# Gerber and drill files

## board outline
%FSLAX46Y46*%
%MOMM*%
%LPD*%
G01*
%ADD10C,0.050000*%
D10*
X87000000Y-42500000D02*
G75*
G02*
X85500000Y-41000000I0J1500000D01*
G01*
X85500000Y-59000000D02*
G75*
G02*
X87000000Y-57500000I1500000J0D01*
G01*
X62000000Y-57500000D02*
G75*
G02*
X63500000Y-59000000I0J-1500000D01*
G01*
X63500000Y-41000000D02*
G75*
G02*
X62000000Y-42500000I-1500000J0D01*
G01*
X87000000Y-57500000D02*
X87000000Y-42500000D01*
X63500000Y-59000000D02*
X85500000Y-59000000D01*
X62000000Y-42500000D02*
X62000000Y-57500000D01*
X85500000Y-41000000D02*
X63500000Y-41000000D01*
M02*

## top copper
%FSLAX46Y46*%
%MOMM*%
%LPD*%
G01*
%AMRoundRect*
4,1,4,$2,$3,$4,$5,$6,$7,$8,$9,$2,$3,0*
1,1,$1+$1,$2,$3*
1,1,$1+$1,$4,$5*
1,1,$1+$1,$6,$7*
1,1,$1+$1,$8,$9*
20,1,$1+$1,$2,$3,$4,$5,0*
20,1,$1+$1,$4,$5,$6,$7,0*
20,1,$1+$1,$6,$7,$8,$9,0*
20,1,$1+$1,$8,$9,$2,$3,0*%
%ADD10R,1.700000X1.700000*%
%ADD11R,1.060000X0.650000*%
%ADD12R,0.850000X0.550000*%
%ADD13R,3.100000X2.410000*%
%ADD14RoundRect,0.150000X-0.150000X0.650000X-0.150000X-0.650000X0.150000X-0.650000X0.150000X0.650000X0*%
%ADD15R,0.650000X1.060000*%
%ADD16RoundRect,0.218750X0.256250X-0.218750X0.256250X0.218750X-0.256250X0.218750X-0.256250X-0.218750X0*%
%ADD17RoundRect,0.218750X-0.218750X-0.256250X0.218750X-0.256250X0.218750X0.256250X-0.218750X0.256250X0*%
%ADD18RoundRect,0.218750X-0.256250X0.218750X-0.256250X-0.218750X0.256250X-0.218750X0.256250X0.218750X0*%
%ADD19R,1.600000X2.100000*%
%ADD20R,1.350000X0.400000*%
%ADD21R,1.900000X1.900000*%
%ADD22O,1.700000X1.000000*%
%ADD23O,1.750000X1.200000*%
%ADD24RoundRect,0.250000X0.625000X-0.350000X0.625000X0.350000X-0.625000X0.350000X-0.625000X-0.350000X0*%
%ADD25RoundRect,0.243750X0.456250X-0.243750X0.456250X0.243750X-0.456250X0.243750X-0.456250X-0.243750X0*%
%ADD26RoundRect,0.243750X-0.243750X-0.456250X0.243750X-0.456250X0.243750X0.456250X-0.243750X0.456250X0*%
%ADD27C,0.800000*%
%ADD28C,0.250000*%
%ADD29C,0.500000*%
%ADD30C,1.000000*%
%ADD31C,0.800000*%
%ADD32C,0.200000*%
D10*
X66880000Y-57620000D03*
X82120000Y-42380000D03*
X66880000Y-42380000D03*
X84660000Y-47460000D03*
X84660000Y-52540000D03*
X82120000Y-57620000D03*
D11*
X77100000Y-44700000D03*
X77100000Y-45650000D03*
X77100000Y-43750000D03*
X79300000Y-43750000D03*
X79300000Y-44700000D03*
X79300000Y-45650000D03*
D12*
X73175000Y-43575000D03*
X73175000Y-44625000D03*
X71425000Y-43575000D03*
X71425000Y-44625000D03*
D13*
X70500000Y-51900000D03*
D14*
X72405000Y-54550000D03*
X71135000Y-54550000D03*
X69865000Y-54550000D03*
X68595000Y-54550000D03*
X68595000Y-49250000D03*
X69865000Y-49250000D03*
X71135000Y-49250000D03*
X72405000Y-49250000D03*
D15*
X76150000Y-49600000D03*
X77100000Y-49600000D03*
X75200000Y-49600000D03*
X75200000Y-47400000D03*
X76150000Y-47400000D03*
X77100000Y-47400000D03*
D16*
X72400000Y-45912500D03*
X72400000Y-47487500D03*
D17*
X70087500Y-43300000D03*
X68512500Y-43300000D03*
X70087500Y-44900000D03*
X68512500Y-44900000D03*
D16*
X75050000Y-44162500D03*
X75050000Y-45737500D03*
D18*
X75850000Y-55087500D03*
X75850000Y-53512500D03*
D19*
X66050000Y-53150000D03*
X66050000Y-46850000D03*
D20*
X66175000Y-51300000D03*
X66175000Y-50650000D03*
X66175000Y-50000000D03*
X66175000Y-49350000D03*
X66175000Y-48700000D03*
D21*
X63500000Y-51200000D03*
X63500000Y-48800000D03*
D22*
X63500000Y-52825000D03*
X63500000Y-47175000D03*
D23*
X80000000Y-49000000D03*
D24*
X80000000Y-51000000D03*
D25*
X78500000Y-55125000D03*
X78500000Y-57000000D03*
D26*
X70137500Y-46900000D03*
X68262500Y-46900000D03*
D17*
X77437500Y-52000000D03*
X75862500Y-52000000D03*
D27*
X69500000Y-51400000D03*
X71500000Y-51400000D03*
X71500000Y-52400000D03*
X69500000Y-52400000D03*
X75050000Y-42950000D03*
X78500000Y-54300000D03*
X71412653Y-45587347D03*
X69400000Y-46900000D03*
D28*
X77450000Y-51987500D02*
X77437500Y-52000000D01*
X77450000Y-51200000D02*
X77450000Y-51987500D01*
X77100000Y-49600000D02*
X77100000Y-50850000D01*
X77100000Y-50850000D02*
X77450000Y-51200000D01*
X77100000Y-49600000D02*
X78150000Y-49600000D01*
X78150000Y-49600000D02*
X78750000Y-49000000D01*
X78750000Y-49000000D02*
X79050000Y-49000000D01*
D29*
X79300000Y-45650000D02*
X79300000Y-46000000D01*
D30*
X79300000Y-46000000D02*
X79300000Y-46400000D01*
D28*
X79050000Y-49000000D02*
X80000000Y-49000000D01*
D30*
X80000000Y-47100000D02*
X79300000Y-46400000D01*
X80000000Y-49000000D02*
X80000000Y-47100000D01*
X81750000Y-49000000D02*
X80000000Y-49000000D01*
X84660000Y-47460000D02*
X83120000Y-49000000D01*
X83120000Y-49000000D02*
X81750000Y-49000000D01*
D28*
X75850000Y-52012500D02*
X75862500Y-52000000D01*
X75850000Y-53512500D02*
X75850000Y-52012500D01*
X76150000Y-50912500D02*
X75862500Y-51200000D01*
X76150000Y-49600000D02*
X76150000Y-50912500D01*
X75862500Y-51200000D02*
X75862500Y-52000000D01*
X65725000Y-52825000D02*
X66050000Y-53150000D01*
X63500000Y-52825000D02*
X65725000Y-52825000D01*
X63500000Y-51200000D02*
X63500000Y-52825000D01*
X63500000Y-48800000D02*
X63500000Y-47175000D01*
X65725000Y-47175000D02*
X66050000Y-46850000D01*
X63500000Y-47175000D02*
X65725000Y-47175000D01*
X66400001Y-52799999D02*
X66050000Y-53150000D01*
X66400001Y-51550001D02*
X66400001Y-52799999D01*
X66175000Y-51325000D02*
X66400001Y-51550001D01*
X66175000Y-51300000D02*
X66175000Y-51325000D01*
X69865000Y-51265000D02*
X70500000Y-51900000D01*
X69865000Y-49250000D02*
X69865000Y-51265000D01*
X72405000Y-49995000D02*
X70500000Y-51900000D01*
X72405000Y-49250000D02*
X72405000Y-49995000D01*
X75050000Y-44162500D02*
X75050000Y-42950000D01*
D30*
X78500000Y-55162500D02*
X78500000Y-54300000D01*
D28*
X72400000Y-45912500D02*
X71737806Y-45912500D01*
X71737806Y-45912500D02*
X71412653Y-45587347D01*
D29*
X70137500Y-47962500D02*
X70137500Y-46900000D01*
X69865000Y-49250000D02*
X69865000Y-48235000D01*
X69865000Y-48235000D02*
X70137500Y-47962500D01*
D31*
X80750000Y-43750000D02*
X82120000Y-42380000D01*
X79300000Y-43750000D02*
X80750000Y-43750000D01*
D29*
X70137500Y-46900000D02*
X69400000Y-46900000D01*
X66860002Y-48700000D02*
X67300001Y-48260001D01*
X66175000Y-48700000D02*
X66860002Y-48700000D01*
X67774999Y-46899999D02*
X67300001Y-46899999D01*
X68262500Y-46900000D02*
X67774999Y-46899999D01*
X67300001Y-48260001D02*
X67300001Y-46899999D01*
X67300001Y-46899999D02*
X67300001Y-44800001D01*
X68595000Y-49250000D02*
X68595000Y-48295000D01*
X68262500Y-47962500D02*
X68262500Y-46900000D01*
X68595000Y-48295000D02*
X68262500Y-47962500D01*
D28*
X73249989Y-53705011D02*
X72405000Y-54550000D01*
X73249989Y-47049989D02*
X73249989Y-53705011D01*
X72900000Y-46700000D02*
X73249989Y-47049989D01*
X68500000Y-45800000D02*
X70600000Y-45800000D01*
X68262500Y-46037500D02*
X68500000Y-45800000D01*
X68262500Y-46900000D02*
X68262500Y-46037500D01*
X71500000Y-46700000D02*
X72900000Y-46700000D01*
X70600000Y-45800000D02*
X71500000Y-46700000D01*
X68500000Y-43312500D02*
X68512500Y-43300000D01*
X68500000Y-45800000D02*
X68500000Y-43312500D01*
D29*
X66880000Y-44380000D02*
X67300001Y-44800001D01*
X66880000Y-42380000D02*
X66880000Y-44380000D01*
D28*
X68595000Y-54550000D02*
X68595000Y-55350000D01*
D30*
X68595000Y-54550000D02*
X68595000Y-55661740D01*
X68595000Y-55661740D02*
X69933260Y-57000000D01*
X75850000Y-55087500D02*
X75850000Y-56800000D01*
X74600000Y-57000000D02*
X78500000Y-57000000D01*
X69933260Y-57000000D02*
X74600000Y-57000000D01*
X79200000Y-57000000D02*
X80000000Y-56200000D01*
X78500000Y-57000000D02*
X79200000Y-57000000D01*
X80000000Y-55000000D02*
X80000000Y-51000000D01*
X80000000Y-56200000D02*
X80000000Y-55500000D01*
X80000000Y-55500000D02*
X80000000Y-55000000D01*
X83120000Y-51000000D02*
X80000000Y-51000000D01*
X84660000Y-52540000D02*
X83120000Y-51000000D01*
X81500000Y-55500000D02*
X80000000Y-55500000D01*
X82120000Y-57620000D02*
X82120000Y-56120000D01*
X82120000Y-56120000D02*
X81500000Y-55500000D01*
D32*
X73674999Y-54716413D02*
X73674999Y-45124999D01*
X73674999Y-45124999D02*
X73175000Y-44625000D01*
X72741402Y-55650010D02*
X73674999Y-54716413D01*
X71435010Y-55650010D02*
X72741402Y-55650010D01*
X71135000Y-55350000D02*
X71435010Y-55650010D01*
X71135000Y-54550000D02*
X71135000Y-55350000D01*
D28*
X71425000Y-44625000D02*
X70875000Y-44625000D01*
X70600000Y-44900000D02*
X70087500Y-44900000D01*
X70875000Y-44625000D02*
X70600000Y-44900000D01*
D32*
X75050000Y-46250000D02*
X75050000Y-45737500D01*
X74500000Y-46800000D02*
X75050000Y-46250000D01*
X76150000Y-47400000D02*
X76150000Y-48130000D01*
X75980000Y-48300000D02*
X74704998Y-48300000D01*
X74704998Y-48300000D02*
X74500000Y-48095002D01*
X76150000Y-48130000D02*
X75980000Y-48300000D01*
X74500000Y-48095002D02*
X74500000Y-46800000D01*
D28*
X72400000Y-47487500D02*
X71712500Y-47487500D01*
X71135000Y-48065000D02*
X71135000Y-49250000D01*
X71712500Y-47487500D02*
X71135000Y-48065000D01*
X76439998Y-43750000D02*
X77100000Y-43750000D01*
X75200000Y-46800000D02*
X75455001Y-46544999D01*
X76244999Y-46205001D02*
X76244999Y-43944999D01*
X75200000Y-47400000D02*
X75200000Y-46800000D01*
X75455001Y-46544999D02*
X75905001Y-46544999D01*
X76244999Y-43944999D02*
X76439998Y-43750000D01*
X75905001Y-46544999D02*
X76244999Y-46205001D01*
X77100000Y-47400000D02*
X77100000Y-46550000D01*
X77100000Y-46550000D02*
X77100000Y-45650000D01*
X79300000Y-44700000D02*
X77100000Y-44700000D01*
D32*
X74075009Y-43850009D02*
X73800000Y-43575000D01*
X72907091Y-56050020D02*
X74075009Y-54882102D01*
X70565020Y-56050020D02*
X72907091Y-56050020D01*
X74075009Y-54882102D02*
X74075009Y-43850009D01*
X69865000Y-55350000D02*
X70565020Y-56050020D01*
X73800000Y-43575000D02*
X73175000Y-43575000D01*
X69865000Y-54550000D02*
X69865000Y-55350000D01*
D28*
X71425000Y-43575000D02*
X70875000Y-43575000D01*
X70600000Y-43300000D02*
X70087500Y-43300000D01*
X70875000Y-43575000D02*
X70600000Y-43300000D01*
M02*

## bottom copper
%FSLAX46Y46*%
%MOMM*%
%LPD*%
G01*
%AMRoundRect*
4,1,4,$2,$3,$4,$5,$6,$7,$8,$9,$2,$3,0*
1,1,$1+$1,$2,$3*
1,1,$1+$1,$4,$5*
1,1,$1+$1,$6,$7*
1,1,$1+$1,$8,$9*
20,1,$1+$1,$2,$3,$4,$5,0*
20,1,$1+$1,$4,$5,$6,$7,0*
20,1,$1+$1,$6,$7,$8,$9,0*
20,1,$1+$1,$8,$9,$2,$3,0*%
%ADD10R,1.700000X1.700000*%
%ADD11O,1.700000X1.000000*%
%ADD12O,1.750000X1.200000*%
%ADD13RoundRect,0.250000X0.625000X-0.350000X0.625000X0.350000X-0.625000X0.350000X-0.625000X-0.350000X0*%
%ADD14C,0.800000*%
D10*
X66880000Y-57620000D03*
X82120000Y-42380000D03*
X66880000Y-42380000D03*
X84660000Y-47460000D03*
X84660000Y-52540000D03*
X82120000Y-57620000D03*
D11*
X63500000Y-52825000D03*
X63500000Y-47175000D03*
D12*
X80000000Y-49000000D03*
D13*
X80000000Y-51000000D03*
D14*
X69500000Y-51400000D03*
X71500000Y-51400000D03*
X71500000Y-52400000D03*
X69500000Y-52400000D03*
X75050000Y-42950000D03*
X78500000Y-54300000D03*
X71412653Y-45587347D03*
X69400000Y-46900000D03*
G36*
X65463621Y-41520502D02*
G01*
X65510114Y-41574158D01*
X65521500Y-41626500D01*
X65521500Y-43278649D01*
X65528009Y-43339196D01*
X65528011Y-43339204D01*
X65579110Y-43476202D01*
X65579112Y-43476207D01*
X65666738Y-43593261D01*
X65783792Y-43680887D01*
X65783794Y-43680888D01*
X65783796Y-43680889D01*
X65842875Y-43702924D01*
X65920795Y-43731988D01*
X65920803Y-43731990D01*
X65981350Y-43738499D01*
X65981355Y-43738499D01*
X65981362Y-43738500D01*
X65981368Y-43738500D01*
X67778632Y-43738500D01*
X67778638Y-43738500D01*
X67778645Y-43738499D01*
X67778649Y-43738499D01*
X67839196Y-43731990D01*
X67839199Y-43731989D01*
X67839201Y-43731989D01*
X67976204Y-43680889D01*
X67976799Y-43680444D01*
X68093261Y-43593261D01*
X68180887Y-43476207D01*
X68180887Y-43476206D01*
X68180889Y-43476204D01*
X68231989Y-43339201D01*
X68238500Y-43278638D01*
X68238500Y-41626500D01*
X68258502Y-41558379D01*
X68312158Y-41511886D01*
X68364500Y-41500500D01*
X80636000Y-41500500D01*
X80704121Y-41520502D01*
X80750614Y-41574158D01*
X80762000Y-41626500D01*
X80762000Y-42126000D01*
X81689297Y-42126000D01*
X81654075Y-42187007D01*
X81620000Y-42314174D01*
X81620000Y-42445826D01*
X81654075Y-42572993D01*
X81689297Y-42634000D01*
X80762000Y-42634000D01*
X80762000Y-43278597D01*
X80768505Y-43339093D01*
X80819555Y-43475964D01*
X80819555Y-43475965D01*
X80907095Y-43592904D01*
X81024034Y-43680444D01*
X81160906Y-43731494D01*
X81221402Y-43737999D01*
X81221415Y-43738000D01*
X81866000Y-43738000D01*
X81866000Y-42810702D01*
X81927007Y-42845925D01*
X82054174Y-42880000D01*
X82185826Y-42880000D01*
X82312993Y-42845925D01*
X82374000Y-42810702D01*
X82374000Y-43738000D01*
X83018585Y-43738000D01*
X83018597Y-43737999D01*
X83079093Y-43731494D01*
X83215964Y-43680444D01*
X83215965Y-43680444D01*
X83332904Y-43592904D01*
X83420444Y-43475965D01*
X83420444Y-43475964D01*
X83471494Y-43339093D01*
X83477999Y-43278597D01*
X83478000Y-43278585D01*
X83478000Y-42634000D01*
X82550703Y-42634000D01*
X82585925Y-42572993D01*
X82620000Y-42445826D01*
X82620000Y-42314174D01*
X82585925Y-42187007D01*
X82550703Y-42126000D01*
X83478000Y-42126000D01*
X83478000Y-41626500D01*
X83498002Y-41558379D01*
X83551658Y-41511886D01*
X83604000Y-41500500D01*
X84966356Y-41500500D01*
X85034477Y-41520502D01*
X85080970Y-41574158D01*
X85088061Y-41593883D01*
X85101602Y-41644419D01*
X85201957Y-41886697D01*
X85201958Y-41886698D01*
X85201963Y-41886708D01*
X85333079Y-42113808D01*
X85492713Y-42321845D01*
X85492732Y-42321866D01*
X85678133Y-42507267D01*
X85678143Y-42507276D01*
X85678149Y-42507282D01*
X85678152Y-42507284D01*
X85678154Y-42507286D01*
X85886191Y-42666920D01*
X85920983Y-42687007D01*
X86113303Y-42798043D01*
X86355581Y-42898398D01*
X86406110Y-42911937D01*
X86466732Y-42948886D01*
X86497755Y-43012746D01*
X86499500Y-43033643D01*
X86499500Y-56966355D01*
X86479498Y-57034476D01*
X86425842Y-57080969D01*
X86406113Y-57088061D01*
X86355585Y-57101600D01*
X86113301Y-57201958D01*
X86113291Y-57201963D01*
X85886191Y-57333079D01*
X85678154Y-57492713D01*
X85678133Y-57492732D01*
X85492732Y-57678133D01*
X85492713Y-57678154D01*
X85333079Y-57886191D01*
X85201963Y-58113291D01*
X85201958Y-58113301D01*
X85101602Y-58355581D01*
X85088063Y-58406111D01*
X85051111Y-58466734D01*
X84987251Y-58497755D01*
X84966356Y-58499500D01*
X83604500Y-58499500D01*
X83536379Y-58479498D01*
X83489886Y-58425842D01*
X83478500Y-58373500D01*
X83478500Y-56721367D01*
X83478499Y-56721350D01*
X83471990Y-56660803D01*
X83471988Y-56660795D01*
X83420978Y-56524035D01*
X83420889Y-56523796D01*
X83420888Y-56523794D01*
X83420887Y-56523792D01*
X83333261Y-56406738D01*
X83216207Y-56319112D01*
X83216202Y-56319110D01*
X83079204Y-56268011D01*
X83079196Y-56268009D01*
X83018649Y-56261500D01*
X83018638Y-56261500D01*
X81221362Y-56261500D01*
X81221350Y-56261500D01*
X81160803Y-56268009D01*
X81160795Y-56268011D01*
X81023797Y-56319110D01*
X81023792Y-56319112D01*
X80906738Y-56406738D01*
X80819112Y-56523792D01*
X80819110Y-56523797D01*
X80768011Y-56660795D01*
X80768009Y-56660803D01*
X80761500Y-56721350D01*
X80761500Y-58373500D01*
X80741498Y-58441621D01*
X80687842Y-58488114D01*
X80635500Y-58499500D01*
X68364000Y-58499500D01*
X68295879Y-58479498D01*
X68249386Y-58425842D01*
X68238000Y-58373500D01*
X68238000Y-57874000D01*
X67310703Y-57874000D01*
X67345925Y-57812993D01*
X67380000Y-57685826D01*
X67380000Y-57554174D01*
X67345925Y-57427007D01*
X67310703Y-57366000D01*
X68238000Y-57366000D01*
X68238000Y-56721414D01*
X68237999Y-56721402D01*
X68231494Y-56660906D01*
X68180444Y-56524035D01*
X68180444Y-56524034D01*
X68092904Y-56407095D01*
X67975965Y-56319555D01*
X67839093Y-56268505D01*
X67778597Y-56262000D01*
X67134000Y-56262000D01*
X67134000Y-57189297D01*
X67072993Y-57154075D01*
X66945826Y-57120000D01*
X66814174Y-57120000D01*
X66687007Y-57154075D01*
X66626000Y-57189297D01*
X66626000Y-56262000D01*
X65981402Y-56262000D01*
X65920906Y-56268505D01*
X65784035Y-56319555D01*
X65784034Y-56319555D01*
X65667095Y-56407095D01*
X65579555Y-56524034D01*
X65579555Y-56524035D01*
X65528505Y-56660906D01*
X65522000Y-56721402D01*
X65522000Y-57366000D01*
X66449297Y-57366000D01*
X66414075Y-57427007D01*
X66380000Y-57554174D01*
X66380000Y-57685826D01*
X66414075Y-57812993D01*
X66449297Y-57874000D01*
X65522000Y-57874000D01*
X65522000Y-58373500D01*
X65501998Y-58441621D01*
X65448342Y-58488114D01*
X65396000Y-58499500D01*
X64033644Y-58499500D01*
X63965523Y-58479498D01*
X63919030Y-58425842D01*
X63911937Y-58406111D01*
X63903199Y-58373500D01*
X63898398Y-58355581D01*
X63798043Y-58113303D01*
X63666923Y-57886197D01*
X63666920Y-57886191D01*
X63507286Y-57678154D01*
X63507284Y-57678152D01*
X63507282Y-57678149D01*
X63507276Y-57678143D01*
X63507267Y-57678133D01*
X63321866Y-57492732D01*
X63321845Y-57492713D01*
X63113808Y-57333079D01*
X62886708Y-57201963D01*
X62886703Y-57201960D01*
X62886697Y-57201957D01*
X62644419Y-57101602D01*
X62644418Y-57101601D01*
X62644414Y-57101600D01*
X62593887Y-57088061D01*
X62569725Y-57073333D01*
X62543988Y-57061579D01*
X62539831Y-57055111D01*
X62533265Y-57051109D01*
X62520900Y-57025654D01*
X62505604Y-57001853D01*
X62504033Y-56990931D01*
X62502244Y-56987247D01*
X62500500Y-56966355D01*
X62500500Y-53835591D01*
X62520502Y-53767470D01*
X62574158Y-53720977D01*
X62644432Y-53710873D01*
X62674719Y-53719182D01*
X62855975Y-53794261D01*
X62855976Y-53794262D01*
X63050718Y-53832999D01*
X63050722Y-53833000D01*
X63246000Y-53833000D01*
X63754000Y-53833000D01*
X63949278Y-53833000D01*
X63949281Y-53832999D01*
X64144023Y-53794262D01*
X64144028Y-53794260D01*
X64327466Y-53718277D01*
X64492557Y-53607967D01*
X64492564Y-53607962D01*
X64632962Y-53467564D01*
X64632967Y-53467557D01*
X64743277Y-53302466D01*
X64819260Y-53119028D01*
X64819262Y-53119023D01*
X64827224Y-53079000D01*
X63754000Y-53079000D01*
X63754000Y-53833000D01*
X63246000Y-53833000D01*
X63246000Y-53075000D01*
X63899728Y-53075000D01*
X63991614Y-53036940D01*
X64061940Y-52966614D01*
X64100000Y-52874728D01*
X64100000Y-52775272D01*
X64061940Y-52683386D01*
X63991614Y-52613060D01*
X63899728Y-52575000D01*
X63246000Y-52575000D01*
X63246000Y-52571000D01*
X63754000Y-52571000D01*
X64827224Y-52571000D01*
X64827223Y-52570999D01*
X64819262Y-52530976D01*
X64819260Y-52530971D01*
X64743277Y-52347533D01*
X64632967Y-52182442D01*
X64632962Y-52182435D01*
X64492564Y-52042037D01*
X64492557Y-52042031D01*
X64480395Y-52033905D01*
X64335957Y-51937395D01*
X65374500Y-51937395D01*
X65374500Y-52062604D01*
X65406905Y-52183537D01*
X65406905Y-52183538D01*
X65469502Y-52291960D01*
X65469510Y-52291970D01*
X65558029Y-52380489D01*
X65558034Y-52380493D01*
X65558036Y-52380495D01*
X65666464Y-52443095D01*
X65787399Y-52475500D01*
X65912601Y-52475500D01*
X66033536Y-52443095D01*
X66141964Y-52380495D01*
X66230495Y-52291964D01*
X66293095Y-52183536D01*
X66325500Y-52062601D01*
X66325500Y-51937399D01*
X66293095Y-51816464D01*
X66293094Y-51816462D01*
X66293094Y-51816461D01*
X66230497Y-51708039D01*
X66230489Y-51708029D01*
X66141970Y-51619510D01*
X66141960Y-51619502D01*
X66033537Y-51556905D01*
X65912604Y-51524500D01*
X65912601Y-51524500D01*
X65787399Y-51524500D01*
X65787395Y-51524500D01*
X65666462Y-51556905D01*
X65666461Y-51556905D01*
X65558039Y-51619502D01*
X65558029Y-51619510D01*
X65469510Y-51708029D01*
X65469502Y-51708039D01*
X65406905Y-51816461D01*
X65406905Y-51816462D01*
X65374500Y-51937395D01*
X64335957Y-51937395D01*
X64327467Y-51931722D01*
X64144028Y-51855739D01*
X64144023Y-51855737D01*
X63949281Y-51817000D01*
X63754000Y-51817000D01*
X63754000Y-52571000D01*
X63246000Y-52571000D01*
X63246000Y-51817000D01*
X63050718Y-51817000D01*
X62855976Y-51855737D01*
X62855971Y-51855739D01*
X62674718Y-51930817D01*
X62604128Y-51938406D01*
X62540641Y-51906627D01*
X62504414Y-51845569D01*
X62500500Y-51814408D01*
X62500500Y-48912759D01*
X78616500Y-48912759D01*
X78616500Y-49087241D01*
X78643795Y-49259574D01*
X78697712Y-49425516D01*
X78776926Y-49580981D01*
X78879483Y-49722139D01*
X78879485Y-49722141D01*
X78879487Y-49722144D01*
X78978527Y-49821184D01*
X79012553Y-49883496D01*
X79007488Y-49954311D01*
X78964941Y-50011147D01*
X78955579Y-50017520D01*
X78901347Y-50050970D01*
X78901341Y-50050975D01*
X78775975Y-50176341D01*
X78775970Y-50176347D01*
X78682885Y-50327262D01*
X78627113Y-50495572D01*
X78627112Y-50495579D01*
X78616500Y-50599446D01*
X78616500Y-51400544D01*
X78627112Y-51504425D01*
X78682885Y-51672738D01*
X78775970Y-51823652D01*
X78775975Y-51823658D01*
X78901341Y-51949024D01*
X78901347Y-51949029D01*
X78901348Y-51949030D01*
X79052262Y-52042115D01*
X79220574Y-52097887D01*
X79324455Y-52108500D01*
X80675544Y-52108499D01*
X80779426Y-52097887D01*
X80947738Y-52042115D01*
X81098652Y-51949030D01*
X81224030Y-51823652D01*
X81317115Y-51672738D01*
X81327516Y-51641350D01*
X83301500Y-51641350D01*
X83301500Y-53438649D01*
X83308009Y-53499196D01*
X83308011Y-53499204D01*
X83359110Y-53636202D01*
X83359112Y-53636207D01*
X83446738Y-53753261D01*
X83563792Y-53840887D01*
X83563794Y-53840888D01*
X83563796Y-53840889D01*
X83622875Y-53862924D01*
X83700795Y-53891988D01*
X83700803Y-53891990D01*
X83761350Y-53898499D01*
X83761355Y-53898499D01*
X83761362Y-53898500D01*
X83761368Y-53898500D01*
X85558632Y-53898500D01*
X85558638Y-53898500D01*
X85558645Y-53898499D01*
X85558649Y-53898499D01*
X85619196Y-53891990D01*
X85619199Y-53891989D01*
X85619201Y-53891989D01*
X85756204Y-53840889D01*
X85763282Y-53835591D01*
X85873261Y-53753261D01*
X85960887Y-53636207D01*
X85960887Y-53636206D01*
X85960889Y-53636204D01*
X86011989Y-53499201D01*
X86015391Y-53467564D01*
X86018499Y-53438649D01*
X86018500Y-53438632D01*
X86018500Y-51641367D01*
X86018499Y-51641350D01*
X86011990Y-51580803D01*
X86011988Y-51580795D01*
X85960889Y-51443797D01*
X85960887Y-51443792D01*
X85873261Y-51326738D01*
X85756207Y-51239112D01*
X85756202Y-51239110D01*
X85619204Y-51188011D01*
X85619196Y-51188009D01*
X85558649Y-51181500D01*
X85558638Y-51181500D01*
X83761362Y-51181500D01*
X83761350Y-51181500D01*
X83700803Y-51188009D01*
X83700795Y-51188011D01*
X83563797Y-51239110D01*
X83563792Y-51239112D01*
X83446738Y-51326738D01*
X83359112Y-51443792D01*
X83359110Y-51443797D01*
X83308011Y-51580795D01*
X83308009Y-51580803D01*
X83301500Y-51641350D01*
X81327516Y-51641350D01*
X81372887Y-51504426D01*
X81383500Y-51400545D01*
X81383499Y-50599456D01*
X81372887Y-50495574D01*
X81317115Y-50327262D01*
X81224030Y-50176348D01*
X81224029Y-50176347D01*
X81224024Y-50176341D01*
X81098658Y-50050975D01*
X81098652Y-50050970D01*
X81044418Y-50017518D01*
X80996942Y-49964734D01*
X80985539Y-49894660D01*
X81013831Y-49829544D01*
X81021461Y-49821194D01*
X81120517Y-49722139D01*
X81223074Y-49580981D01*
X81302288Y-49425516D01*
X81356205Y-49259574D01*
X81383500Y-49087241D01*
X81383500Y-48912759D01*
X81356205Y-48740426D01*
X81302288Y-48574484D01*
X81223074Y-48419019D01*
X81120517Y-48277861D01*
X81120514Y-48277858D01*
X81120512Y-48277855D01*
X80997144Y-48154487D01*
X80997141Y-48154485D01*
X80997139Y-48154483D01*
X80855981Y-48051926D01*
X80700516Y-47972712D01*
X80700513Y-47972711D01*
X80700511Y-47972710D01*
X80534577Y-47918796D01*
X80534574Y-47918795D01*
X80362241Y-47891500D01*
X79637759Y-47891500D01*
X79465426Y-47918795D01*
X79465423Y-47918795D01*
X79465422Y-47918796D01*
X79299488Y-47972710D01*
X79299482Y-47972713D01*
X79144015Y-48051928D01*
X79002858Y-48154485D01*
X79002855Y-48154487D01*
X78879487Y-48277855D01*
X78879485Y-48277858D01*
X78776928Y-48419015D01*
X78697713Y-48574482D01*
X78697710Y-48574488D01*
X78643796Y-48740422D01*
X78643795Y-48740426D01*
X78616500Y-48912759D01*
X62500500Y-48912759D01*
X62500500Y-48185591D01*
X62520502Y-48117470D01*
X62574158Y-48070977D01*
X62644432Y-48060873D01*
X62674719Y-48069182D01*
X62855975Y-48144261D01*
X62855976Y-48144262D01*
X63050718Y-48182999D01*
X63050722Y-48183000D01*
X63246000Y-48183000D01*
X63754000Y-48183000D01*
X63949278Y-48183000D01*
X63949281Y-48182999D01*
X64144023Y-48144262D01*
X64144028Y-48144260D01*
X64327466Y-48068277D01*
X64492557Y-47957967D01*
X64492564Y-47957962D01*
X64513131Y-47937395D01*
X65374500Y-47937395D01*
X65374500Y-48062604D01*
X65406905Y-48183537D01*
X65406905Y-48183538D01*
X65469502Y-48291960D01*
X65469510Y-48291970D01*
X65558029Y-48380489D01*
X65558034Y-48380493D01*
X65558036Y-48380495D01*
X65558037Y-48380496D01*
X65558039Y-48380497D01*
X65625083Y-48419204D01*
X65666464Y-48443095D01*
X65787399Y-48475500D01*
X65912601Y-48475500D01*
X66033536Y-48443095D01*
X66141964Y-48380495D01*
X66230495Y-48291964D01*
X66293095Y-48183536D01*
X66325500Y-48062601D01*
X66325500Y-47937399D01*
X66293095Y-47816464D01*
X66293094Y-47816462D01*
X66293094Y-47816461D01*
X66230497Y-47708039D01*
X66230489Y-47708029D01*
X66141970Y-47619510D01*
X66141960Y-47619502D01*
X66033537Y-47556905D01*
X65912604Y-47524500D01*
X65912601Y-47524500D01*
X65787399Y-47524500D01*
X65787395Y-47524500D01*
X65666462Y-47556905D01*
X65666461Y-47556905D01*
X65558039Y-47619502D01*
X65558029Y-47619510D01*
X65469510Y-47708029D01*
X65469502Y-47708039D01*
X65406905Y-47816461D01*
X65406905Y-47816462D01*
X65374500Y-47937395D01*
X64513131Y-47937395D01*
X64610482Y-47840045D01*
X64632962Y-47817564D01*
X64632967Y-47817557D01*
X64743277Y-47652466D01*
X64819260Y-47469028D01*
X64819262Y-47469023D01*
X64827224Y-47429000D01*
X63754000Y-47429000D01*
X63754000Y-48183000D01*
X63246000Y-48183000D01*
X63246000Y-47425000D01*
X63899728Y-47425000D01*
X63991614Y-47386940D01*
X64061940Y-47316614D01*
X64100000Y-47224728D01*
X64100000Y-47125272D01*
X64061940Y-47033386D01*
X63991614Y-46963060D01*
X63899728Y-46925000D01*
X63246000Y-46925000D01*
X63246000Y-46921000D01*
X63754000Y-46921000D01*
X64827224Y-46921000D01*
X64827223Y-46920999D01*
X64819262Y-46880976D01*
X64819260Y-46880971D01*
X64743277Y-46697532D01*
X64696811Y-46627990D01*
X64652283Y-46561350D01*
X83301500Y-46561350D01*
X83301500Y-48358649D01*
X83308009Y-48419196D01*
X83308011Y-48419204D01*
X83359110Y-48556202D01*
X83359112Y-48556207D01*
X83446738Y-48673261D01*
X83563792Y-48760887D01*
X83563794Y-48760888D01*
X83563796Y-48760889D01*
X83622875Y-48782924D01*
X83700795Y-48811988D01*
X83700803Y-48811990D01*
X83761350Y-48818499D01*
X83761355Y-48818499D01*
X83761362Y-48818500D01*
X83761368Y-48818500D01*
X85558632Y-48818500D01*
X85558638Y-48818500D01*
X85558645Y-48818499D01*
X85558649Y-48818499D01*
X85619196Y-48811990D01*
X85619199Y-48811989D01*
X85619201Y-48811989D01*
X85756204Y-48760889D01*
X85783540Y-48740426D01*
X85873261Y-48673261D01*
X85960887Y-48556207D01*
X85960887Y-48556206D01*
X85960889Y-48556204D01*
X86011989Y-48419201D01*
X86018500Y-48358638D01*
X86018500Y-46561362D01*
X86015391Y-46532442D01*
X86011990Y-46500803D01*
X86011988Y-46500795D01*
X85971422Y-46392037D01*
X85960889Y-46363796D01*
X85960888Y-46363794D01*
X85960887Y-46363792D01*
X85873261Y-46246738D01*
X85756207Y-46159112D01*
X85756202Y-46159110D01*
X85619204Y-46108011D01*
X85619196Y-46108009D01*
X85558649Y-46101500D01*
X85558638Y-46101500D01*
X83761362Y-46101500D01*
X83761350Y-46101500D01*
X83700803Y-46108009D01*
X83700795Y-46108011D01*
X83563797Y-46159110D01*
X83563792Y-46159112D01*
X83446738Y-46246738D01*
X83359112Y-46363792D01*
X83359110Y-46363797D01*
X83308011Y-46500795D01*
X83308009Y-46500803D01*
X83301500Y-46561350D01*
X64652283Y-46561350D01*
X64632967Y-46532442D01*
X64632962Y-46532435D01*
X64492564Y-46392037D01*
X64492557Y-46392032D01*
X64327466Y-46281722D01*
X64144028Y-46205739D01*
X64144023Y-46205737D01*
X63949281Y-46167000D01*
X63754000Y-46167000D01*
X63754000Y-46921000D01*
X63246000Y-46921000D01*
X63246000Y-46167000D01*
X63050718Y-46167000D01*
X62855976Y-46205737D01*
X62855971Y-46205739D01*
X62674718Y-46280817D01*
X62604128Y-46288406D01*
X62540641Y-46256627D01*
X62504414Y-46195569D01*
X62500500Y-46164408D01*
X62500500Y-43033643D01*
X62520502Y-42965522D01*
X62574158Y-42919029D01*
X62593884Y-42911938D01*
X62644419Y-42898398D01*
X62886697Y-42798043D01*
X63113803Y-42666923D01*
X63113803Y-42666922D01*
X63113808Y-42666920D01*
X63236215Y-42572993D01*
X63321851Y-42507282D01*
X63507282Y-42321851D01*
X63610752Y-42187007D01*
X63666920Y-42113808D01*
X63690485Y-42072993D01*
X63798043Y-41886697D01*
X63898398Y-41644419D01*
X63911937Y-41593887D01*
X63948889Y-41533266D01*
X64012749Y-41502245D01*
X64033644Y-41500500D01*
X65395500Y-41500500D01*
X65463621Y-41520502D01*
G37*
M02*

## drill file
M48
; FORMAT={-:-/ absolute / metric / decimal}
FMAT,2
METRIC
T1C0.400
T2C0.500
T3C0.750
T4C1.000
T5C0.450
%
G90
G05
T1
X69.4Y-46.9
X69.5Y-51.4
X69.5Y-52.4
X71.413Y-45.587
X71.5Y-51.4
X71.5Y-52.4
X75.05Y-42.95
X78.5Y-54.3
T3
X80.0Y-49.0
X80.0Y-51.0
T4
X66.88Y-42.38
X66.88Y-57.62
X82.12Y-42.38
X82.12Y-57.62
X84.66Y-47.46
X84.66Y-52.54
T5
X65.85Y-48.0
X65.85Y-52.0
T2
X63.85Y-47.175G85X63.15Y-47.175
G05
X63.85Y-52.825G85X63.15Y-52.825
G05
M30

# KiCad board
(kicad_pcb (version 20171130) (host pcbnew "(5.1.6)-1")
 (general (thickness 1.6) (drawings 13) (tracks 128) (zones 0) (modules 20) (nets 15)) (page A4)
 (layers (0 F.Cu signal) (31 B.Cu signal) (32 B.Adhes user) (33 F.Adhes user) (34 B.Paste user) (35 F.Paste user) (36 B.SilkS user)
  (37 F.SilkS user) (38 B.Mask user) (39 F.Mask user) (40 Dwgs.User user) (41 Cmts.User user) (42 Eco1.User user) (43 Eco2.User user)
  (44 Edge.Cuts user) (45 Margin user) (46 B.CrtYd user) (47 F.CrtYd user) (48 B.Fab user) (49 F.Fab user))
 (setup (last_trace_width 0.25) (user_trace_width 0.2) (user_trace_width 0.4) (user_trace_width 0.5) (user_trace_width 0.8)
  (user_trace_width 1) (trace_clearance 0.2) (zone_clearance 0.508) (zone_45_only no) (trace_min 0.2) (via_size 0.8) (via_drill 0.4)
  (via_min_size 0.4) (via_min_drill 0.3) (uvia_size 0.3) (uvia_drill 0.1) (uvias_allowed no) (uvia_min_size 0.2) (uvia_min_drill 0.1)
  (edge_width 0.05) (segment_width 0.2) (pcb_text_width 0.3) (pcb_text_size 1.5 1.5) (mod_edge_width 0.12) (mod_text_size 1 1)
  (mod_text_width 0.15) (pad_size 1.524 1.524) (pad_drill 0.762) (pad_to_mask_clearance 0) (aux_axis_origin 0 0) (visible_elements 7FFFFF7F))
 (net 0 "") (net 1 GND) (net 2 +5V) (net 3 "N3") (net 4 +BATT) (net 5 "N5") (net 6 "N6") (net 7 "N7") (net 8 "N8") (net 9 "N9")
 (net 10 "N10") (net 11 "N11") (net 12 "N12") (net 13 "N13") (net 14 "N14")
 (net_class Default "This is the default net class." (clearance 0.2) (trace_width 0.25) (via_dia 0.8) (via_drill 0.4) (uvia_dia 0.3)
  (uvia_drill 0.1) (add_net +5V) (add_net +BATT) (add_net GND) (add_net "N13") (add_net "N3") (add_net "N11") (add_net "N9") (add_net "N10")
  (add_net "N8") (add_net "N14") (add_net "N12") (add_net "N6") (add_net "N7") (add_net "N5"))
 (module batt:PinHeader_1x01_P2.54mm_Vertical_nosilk (layer F.Cu) (at 66.88 57.62 90)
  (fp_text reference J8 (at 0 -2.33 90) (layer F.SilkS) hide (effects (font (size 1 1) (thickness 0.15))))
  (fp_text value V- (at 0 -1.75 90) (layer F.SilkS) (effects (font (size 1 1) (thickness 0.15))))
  (pad 1 thru_hole rect (at 0 0 90) (size 1.7 1.7) (drill 1) (layers *.Cu *.Mask) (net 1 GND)))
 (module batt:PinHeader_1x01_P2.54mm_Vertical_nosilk (layer F.Cu) (at 82.12 42.38 270)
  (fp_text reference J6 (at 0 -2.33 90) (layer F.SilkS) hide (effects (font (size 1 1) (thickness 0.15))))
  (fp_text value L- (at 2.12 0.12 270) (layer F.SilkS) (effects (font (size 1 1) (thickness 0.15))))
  (pad 1 thru_hole rect (at 0 0 270) (size 1.7 1.7) (drill 1) (layers *.Cu *.Mask) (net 1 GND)))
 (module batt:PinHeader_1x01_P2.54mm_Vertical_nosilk (layer F.Cu) (at 66.88 42.38 180)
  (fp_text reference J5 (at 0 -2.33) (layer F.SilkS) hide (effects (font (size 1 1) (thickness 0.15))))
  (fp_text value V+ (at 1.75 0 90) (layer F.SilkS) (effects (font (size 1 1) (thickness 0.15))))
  (pad 1 thru_hole rect (at 0 0 180) (size 1.7 1.7) (drill 1) (layers *.Cu *.Mask) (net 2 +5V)))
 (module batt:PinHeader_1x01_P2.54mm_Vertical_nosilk (layer F.Cu) (at 84.66 47.46)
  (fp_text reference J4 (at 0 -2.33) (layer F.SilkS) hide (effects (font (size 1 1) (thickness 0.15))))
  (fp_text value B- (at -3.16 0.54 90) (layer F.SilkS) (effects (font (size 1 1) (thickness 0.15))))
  (pad 1 thru_hole rect (at 0 0) (size 1.7 1.7) (drill 1) (layers *.Cu *.Mask) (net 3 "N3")))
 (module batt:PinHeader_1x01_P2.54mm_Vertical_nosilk (layer F.Cu) (at 84.66 52.54 180)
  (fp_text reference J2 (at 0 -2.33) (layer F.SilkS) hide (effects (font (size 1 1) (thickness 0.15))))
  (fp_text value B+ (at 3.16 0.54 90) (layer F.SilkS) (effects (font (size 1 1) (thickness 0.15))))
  (pad 1 thru_hole rect (at 0 0 180) (size 1.7 1.7) (drill 1) (layers *.Cu *.Mask) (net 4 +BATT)))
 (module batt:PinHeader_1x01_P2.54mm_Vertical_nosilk (layer F.Cu) (at 82.12 57.62)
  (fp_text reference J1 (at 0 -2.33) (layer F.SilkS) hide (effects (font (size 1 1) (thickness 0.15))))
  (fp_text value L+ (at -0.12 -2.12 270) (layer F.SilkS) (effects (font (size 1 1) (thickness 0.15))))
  (pad 1 thru_hole rect (at 0 0) (size 1.7 1.7) (drill 1) (layers *.Cu *.Mask) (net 4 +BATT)))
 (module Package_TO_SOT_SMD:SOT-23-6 (layer F.Cu) (at 78.2 44.7 180)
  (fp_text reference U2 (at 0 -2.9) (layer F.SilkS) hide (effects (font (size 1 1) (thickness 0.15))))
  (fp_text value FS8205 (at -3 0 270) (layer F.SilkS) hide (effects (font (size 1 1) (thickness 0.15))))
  (pad 5 smd rect (at 1.1 0 180) (size 1.06 0.65) (layers F.Cu F.Paste F.Mask) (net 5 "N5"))
  (pad 6 smd rect (at 1.1 -0.95 180) (size 1.06 0.65) (layers F.Cu F.Paste F.Mask) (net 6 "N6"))
  (pad 4 smd rect (at 1.1 0.95 180) (size 1.06 0.65) (layers F.Cu F.Paste F.Mask) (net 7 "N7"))
  (pad 3 smd rect (at -1.1 0.95 180) (size 1.06 0.65) (layers F.Cu F.Paste F.Mask) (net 1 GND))
  (pad 2 smd rect (at -1.1 0 180) (size 1.06 0.65) (layers F.Cu F.Paste F.Mask) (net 5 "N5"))
  (pad 1 smd rect (at -1.1 -0.95 180) (size 1.06 0.65) (layers F.Cu F.Paste F.Mask) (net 3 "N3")))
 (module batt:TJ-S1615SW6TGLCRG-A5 (layer F.Cu) (at 72.3 44.1 180)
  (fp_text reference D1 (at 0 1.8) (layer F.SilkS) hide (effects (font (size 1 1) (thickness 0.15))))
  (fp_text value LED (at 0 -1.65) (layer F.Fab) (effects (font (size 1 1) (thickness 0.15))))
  (pad 4 smd rect (at -0.875 0.525 180) (size 0.85 0.55) (layers F.Cu F.Paste F.Mask) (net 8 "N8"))
  (pad 2 smd rect (at -0.875 -0.525 180) (size 0.85 0.55) (layers F.Cu F.Paste F.Mask) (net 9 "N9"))
  (pad 3 smd rect (at 0.875 0.525 180) (size 0.85 0.55) (layers F.Cu F.Paste F.Mask) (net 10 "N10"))
  (pad 1 smd rect (at 0.875 -0.525 180) (size 0.85 0.55) (layers F.Cu F.Paste F.Mask) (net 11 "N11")))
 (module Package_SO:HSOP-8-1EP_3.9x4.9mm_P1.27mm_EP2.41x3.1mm (layer F.Cu) (at 70.5 51.9 270)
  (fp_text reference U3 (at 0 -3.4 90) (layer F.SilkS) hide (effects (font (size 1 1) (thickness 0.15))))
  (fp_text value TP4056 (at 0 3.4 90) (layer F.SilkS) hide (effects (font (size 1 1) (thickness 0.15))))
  (pad "" smd roundrect (at 0.6 0.775 270) (size 0.97 1.25) (layers F.Paste) (roundrect_rratio 0.25))
  (pad "" smd roundrect (at 0.6 -0.775 270) (size 0.97 1.25) (layers F.Paste) (roundrect_rratio 0.25))
  (pad "" smd roundrect (at -0.6 0.775 270) (size 0.97 1.25) (layers F.Paste) (roundrect_rratio 0.25))
  (pad "" smd roundrect (at -0.6 -0.775 270) (size 0.97 1.25) (layers F.Paste) (roundrect_rratio 0.25))
  (pad 9 smd rect (at 0 0 270) (size 2.41 3.1) (layers F.Cu F.Mask) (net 1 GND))
  (pad 8 smd roundrect (at 2.65 -1.905 270) (size 1.6 0.6) (layers F.Cu F.Paste F.Mask) (roundrect_rratio 0.25) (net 2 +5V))
  (pad 7 smd roundrect (at 2.65 -0.635 270) (size 1.6 0.6) (layers F.Cu F.Paste F.Mask) (roundrect_rratio 0.25) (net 9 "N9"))
  (pad 6 smd roundrect (at 2.65 0.635 270) (size 1.6 0.6) (layers F.Cu F.Paste F.Mask) (roundrect_rratio 0.25) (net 8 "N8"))
  (pad 5 smd roundrect (at 2.65 1.905 270) (size 1.6 0.6) (layers F.Cu F.Paste F.Mask) (roundrect_rratio 0.25) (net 4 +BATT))
  (pad 4 smd roundrect (at -2.65 1.905 270) (size 1.6 0.6) (layers F.Cu F.Paste F.Mask) (roundrect_rratio 0.25) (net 2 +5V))
  (pad 3 smd roundrect (at -2.65 0.635 270) (size 1.6 0.6) (layers F.Cu F.Paste F.Mask) (roundrect_rratio 0.25) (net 1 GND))
  (pad 2 smd roundrect (at -2.65 -0.635 270) (size 1.6 0.6) (layers F.Cu F.Paste F.Mask) (roundrect_rratio 0.25) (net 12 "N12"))
  (pad 1 smd roundrect (at -2.65 -1.905 270) (size 1.6 0.6) (layers F.Cu F.Paste F.Mask) (roundrect_rratio 0.25) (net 1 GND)))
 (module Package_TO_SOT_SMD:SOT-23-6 (layer F.Cu) (at 76.15 48.5 270)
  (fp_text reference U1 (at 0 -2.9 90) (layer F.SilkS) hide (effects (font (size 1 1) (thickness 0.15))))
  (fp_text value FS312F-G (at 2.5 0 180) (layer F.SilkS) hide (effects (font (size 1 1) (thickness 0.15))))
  (pad 5 smd rect (at 1.1 0 270) (size 1.06 0.65) (layers F.Cu F.Paste F.Mask) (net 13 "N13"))
  (pad 6 smd rect (at 1.1 -0.95 270) (size 1.06 0.65) (layers F.Cu F.Paste F.Mask) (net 3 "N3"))
  (pad 4 smd rect (at 1.1 0.95 270) (size 1.06 0.65) (layers F.Cu F.Paste F.Mask))
  (pad 3 smd rect (at -1.1 0.95 270) (size 1.06 0.65) (layers F.Cu F.Paste F.Mask) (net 7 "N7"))
  (pad 2 smd rect (at -1.1 0 270) (size 1.06 0.65) (layers F.Cu F.Paste F.Mask) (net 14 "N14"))
  (pad 1 smd rect (at -1.1 -0.95 270) (size 1.06 0.65) (layers F.Cu F.Paste F.Mask) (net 6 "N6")))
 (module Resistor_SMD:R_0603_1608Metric (layer F.Cu) (at 72.4 46.7 90)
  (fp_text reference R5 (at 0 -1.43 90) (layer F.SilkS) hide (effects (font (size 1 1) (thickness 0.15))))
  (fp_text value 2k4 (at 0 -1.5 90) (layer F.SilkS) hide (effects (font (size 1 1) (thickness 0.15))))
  (pad 2 smd roundrect (at 0.7875 0 90) (size 0.875 0.95) (layers F.Cu F.Paste F.Mask) (roundrect_rratio 0.25) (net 1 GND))
  (pad 1 smd roundrect (at -0.7875 0 90) (size 0.875 0.95) (layers F.Cu F.Paste F.Mask) (roundrect_rratio 0.25) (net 12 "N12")))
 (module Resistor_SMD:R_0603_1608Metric (layer F.Cu) (at 69.3 43.3)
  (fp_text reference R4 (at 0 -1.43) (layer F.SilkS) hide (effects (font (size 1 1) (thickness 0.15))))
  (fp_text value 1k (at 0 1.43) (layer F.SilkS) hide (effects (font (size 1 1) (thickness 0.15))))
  (pad 2 smd roundrect (at 0.7875 0) (size 0.875 0.95) (layers F.Cu F.Paste F.Mask) (roundrect_rratio 0.25) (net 10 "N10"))
  (pad 1 smd roundrect (at -0.7875 0) (size 0.875 0.95) (layers F.Cu F.Paste F.Mask) (roundrect_rratio 0.25) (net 2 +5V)))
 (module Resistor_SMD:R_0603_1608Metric (layer F.Cu) (at 69.3 44.9)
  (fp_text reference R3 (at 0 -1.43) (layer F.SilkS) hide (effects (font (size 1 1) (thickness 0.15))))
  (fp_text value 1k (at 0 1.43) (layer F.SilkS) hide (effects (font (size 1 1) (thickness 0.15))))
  (pad 2 smd roundrect (at 0.7875 0) (size 0.875 0.95) (layers F.Cu F.Paste F.Mask) (roundrect_rratio 0.25) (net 11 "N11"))
  (pad 1 smd roundrect (at -0.7875 0) (size 0.875 0.95) (layers F.Cu F.Paste F.Mask) (roundrect_rratio 0.25) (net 2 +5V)))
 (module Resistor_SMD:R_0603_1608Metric (layer F.Cu) (at 75.05 44.95 90)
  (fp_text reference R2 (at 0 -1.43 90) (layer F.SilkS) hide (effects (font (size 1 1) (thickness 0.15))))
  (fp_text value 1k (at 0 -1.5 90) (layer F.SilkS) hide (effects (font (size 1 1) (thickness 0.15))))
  (pad 2 smd roundrect (at 0.7875 0 90) (size 0.875 0.95) (layers F.Cu F.Paste F.Mask) (roundrect_rratio 0.25) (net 1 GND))
  (pad 1 smd roundrect (at -0.7875 0 90) (size 0.875 0.95) (layers F.Cu F.Paste F.Mask) (roundrect_rratio 0.25) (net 14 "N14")))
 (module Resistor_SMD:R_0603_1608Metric (layer F.Cu) (at 75.85 54.3 270)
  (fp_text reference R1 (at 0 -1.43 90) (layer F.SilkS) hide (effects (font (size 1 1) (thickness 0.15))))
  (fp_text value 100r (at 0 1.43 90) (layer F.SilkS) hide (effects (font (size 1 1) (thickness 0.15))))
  (pad 2 smd roundrect (at 0.7875 0 270) (size 0.875 0.95) (layers F.Cu F.Paste F.Mask) (roundrect_rratio 0.25) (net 4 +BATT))
  (pad 1 smd roundrect (at -0.7875 0 270) (size 0.875 0.95) (layers F.Cu F.Paste F.Mask) (roundrect_rratio 0.25) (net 13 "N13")))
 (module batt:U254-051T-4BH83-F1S (layer F.Cu) (at 63.5 50 270)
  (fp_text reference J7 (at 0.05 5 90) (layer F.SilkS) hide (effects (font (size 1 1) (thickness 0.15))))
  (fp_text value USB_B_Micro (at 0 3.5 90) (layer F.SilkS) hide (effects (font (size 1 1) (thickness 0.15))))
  (pad 6 smd rect (at 3.15 -2.55 270) (size 2.1 1.6) (layers F.Cu F.Paste F.Mask) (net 1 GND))
  (pad 6 smd rect (at -3.15 -2.55 270) (size 2.1 1.6) (layers F.Cu F.Paste F.Mask) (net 1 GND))
  (pad 5 smd rect (at 1.3 -2.675 270) (size 0.4 1.35) (layers F.Cu F.Paste F.Mask) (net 1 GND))
  (pad 4 smd rect (at 0.65 -2.675 270) (size 0.4 1.35) (layers F.Cu F.Paste F.Mask))
  (pad 3 smd rect (at 0 -2.675 270) (size 0.4 1.35) (layers F.Cu F.Paste F.Mask))
  (pad 2 smd rect (at -0.65 -2.675 270) (size 0.4 1.35) (layers F.Cu F.Paste F.Mask))
  (pad 1 smd rect (at -1.3 -2.675 270) (size 0.4 1.35) (layers F.Cu F.Paste F.Mask) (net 2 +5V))
  (pad "" np_thru_hole circle (at 2 -2.35 270) (size 0.45 0.45) (drill 0.45) (layers *.Cu *.Mask))
  (pad "" np_thru_hole circle (at -2 -2.35 270) (size 0.45 0.45) (drill 0.45) (layers *.Cu *.Mask))
  (pad 6 smd rect (at 1.2 0 270) (size 1.9 1.9) (layers F.Cu F.Paste F.Mask) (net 1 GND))
  (pad 6 smd rect (at -1.2 0 270) (size 1.9 1.9) (layers F.Cu F.Paste F.Mask) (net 1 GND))
  (pad 6 thru_hole oval (at 2.825 0 270) (size 1 1.7) (drill oval 0.5 1.2) (layers *.Cu *.Mask) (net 1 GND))
  (pad 6 thru_hole oval (at -2.825 0 270) (size 1 1.7) (drill oval 0.5 1.2) (layers *.Cu *.Mask) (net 1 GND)))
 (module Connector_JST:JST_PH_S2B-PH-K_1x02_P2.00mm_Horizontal (layer F.Cu) (at 80 51 90)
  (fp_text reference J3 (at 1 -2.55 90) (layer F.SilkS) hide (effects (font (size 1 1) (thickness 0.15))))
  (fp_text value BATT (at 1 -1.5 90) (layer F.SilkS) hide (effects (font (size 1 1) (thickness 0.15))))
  (pad 2 thru_hole oval (at 2 0 90) (size 1.2 1.75) (drill 0.75) (layers *.Cu *.Mask) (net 3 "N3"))
  (pad 1 thru_hole roundrect (at 0 0 90) (size 1.2 1.75) (drill 0.75) (layers *.Cu *.Mask) (roundrect_rratio 0.208333) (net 4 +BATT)))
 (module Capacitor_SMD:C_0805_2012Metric (layer F.Cu) (at 78.5 56.0625 90)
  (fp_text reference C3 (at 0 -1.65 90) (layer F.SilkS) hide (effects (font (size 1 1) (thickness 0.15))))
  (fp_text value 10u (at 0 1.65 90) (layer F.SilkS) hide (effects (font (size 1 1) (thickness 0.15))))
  (pad 2 smd roundrect (at 0.9375 0 90) (size 0.975 1.4) (layers F.Cu F.Paste F.Mask) (roundrect_rratio 0.25) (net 1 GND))
  (pad 1 smd roundrect (at -0.9375 0 90) (size 0.975 1.4) (layers F.Cu F.Paste F.Mask) (roundrect_rratio 0.25) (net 4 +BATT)))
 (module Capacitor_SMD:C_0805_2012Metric (layer F.Cu) (at 69.2 46.9)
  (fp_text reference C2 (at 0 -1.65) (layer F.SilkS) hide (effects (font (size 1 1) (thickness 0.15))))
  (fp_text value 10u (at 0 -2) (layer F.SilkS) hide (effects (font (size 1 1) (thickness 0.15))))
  (pad 2 smd roundrect (at 0.9375 0) (size 0.975 1.4) (layers F.Cu F.Paste F.Mask) (roundrect_rratio 0.25) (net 1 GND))
  (pad 1 smd roundrect (at -0.9375 0) (size 0.975 1.4) (layers F.Cu F.Paste F.Mask) (roundrect_rratio 0.25) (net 2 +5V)))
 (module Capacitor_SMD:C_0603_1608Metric (layer F.Cu) (at 76.65 52)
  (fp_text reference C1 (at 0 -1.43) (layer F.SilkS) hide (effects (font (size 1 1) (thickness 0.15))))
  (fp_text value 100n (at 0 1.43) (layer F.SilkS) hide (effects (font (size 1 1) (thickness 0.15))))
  (pad 2 smd roundrect (at 0.7875 0) (size 0.875 0.95) (layers F.Cu F.Paste F.Mask) (roundrect_rratio 0.25) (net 3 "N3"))
  (pad 1 smd roundrect (at -0.7875 0) (size 0.875 0.95) (layers F.Cu F.Paste F.Mask) (roundrect_rratio 0.25) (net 13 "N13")))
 (gr_arc (start 87 41) (end 85.5 41) (angle -90) (layer Edge.Cuts) (width 0.05))
 (gr_arc (start 87 59) (end 87 57.5) (angle -90) (layer Edge.Cuts) (width 0.05))
 (gr_arc (start 62 59) (end 63.5 59) (angle -90) (layer Edge.Cuts) (width 0.05))
 (gr_arc (start 62 41) (end 62 42.5) (angle -90) (layer Edge.Cuts) (width 0.05))
 (gr_line (start 87 57.5) (end 87 42.5) (layer Edge.Cuts) (width 0.05))
 (gr_line (start 63.5 59) (end 85.5 59) (layer Edge.Cuts) (width 0.05))
 (gr_line (start 62 42.5) (end 62 57.5) (layer Edge.Cuts) (width 0.05))
 (gr_line (start 85.5 41) (end 63.5 41) (layer Edge.Cuts) (width 0.05))
 (segment (start 77.45 51.9875) (end 77.4375 52) (width 0.25) (layer F.Cu) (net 3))
 (segment (start 77.45 51.2) (end 77.45 51.9875) (width 0.25) (layer F.Cu) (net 3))
 (segment (start 77.1 49.6) (end 77.1 50.85) (width 0.25) (layer F.Cu) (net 3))
 (segment (start 77.1 50.85) (end 77.45 51.2) (width 0.25) (layer F.Cu) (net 3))
 (segment (start 77.1 49.6) (end 78.15 49.6) (width 0.25) (layer F.Cu) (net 3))
 (segment (start 78.15 49.6) (end 78.75 49) (width 0.25) (layer F.Cu) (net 3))
 (segment (start 78.75 49) (end 79.05 49) (width 0.25) (layer F.Cu) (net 3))
 (segment (start 79.3 45.65) (end 79.3 46) (width 0.5) (layer F.Cu) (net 3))
 (segment (start 79.3 46) (end 79.3 46.4) (width 1) (layer F.Cu) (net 3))
 (segment (start 79.05 49) (end 80 49) (width 0.25) (layer F.Cu) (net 3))
 (segment (start 80 47.1) (end 79.3 46.4) (width 1) (layer F.Cu) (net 3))
 (segment (start 80 49) (end 80 47.1) (width 1) (layer F.Cu) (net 3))
 (segment (start 81.75 49) (end 80 49) (width 1) (layer F.Cu) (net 3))
 (segment (start 84.66 47.46) (end 83.12 49) (width 1) (layer F.Cu) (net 3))
 (segment (start 83.12 49) (end 81.75 49) (width 1) (layer F.Cu) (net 3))
 (segment (start 75.85 52.0125) (end 75.8625 52) (width 0.25) (layer F.Cu) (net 13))
 (segment (start 75.85 53.5125) (end 75.85 52.0125) (width 0.25) (layer F.Cu) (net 13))
 (segment (start 76.15 50.9125) (end 75.8625 51.2) (width 0.25) (layer F.Cu) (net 13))
 (segment (start 76.15 49.6) (end 76.15 50.9125) (width 0.25) (layer F.Cu) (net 13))
 (segment (start 75.8625 51.2) (end 75.8625 52) (width 0.25) (layer F.Cu) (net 13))
 (via (at 69.5 51.4) (size 0.8) (drill 0.4) (layers F.Cu B.Cu) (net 1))
 (via (at 71.5 51.4) (size 0.8) (drill 0.4) (layers F.Cu B.Cu) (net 1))
 (via (at 71.5 52.4) (size 0.8) (drill 0.4) (layers F.Cu B.Cu) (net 1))
 (via (at 69.5 52.4) (size 0.8) (drill 0.4) (layers F.Cu B.Cu) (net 1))
 (segment (start 65.725 52.825) (end 66.05 53.15) (width 0.25) (layer F.Cu) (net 1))
 (segment (start 63.5 52.825) (end 65.725 52.825) (width 0.25) (layer F.Cu) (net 1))
 (segment (start 63.5 51.2) (end 63.5 52.825) (width 0.25) (layer F.Cu) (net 1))
 (segment (start 63.5 48.8) (end 63.5 47.175) (width 0.25) (layer F.Cu) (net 1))
 (segment (start 65.725 47.175) (end 66.05 46.85) (width 0.25) (layer F.Cu) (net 1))
 (segment (start 63.5 47.175) (end 65.725 47.175) (width 0.25) (layer F.Cu) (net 1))
 (segment (start 66.400001 52.799999) (end 66.05 53.15) (width 0.25) (layer F.Cu) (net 1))
 (segment (start 66.400001 51.550001) (end 66.400001 52.799999) (width 0.25) (layer F.Cu) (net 1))
 (segment (start 66.175 51.325) (end 66.400001 51.550001) (width 0.25) (layer F.Cu) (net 1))
 (segment (start 66.175 51.3) (end 66.175 51.325) (width 0.25) (layer F.Cu) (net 1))
 (segment (start 69.865 51.265) (end 70.5 51.9) (width 0.25) (layer F.Cu) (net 1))
 (segment (start 69.865 49.25) (end 69.865 51.265) (width 0.25) (layer F.Cu) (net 1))
 (segment (start 72.405 49.995) (end 70.5 51.9) (width 0.25) (layer F.Cu) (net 1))
 (segment (start 72.405 49.25) (end 72.405 49.995) (width 0.25) (layer F.Cu) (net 1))
 (via (at 75.05 42.95) (size 0.8) (drill 0.4) (layers F.Cu B.Cu) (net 1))
 (segment (start 75.05 44.1625) (end 75.05 42.95) (width 0.25) (layer F.Cu) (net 1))
 (via (at 78.5 54.3) (size 0.8) (drill 0.4) (layers F.Cu B.Cu) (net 1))
 (segment (start 78.5 55.1625) (end 78.5 54.3) (width 1) (layer F.Cu) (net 1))
 (segment (start 72.4 45.9125) (end 71.737806 45.9125) (width 0.25) (layer F.Cu) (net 1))
 (via (at 71.412653 45.587347) (size 0.8) (drill 0.4) (layers F.Cu B.Cu) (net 1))
 (segment (start 71.737806 45.9125) (end 71.412653 45.587347) (width 0.25) (layer F.Cu) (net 1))
 (segment (start 70.1375 47.9625) (end 70.1375 46.9) (width 0.5) (layer F.Cu) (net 1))
 (segment (start 69.865 49.25) (end 69.865 48.235) (width 0.5) (layer F.Cu) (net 1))
 (segment (start 69.865 48.235) (end 70.1375 47.9625) (width 0.5) (layer F.Cu) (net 1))
 (segment (start 80.75 43.75) (end 82.12 42.38) (width 0.8) (layer F.Cu) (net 1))
 (segment (start 79.3 43.75) (end 80.75 43.75) (width 0.8) (layer F.Cu) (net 1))
 (via (at 69.4 46.9) (size 0.8) (drill 0.4) (layers F.Cu B.Cu) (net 1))
 (segment (start 70.1375 46.9) (end 69.4 46.9) (width 0.5) (layer F.Cu) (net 1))
 (segment (start 66.860002 48.7) (end 67.300001 48.260001) (width 0.5) (layer F.Cu) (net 2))
 (segment (start 66.175 48.7) (end 66.860002 48.7) (width 0.5) (layer F.Cu) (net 2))
 (segment (start 67.774999 46.899999) (end 67.300001 46.899999) (width 0.5) (layer F.Cu) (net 2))
 (segment (start 68.2625 46.9) (end 67.774999 46.899999) (width 0.5) (layer F.Cu) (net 2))
 (segment (start 67.300001 48.260001) (end 67.300001 46.899999) (width 0.5) (layer F.Cu) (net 2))
 (segment (start 67.300001 46.899999) (end 67.300001 44.800001) (width 0.5) (layer F.Cu) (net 2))
 (segment (start 68.595 49.25) (end 68.595 48.295) (width 0.5) (layer F.Cu) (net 2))
 (segment (start 68.2625 47.9625) (end 68.2625 46.9) (width 0.5) (layer F.Cu) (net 2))
 (segment (start 68.595 48.295) (end 68.2625 47.9625) (width 0.5) (layer F.Cu) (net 2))
 (segment (start 73.249989 53.705011) (end 72.405 54.55) (width 0.25) (layer F.Cu) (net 2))
 (segment (start 73.249989 47.049989) (end 73.249989 53.705011) (width 0.25) (layer F.Cu) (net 2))
 (segment (start 72.9 46.7) (end 73.249989 47.049989) (width 0.25) (layer F.Cu) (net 2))
 (segment (start 68.5 45.8) (end 70.6 45.8) (width 0.25) (layer F.Cu) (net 2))
 (segment (start 68.2625 46.0375) (end 68.5 45.8) (width 0.25) (layer F.Cu) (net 2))
 (segment (start 68.2625 46.9) (end 68.2625 46.0375) (width 0.25) (layer F.Cu) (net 2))
 (segment (start 71.5 46.7) (end 72.9 46.7) (width 0.25) (layer F.Cu) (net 2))
 (segment (start 70.6 45.8) (end 71.5 46.7) (width 0.25) (layer F.Cu) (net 2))
 (segment (start 68.5 43.3125) (end 68.5125 43.3) (width 0.25) (layer F.Cu) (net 2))
 (segment (start 68.5 45.8) (end 68.5 43.3125) (width 0.25) (layer F.Cu) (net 2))
 (segment (start 66.88 44.38) (end 67.300001 44.800001) (width 0.5) (layer F.Cu) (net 2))
 (segment (start 66.88 42.38) (end 66.88 44.38) (width 0.5) (layer F.Cu) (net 2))
 (segment (start 68.595 54.55) (end 68.595 55.35) (width 0.25) (layer F.Cu) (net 4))
 (segment (start 68.595 54.55) (end 68.595 55.66174) (width 1) (layer F.Cu) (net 4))
 (segment (start 68.595 55.66174) (end 69.93326 57) (width 1) (layer F.Cu) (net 4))
 (segment (start 75.85 55.0875) (end 75.85 56.8) (width 1) (layer F.Cu) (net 4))
 (segment (start 74.6 57) (end 78.5 57) (width 1) (layer F.Cu) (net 4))
 (segment (start 69.93326 57) (end 74.6 57) (width 1) (layer F.Cu) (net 4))
 (segment (start 79.2 57) (end 80 56.2) (width 1) (layer F.Cu) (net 4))
 (segment (start 78.5 57) (end 79.2 57) (width 1) (layer F.Cu) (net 4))
 (segment (start 80 55) (end 80 51) (width 1) (layer F.Cu) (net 4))
 (segment (start 80 56.2) (end 80 55.5) (width 1) (layer F.Cu) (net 4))
 (segment (start 80 55.5) (end 80 55) (width 1) (layer F.Cu) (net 4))
 (segment (start 83.12 51) (end 80 51) (width 1) (layer F.Cu) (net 4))
 (segment (start 84.66 52.54) (end 83.12 51) (width 1) (layer F.Cu) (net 4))
 (segment (start 81.5 55.5) (end 80 55.5) (width 1) (layer F.Cu) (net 4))
 (segment (start 82.12 57.62) (end 82.12 56.12) (width 1) (layer F.Cu) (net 4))
 (segment (start 82.12 56.12) (end 81.5 55.5) (width 1) (layer F.Cu) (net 4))
 (segment (start 73.674999 54.716413) (end 73.674999 45.124999) (width 0.2) (layer F.Cu) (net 9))
 (segment (start 73.674999 45.124999) (end 73.175 44.625) (width 0.2) (layer F.Cu) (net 9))
 (segment (start 72.741402 55.65001) (end 73.674999 54.716413) (width 0.2) (layer F.Cu) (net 9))
 (segment (start 71.43501 55.65001) (end 72.741402 55.65001) (width 0.2) (layer F.Cu) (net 9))
 (segment (start 71.135 55.35) (end 71.43501 55.65001) (width 0.2) (layer F.Cu) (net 9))
 (segment (start 71.135 54.55) (end 71.135 55.35) (width 0.2) (layer F.Cu) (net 9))
 (segment (start 71.425 44.625) (end 70.875 44.625) (width 0.25) (layer F.Cu) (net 11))
 (segment (start 70.6 44.9) (end 70.0875 44.9) (width 0.25) (layer F.Cu) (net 11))
 (segment (start 70.875 44.625) (end 70.6 44.9) (width 0.25) (layer F.Cu) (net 11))
 (segment (start 75.05 46.25) (end 75.05 45.7375) (width 0.2) (layer F.Cu) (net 14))
 (segment (start 74.5 46.8) (end 75.05 46.25) (width 0.2) (layer F.Cu) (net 14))
 (segment (start 76.15 47.4) (end 76.15 48.13) (width 0.2) (layer F.Cu) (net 14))
 (segment (start 75.98 48.3) (end 74.704998 48.3) (width 0.2) (layer F.Cu) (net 14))
 (segment (start 74.704998 48.3) (end 74.5 48.095002) (width 0.2) (layer F.Cu) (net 14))
 (segment (start 76.15 48.13) (end 75.98 48.3) (width 0.2) (layer F.Cu) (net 14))
 (segment (start 74.5 48.095002) (end 74.5 46.8) (width 0.2) (layer F.Cu) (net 14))
 (segment (start 72.4 47.4875) (end 71.7125 47.4875) (width 0.25) (layer F.Cu) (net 12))
 (segment (start 71.135 48.065) (end 71.135 49.25) (width 0.25) (layer F.Cu) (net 12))
 (segment (start 71.7125 47.4875) (end 71.135 48.065) (width 0.25) (layer F.Cu) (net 12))
 (segment (start 76.439998 43.75) (end 77.1 43.75) (width 0.25) (layer F.Cu) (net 7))
 (segment (start 75.2 46.8) (end 75.455001 46.544999) (width 0.25) (layer F.Cu) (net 7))
 (segment (start 76.244999 46.205001) (end 76.244999 43.944999) (width 0.25) (layer F.Cu) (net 7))
 (segment (start 75.2 47.4) (end 75.2 46.8) (width 0.25) (layer F.Cu) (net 7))
 (segment (start 75.455001 46.544999) (end 75.905001 46.544999) (width 0.25) (layer F.Cu) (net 7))
 (segment (start 76.244999 43.944999) (end 76.439998 43.75) (width 0.25) (layer F.Cu) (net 7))
 (segment (start 75.905001 46.544999) (end 76.244999 46.205001) (width 0.25) (layer F.Cu) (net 7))
 (segment (start 77.1 47.4) (end 77.1 46.55) (width 0.25) (layer F.Cu) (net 6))
 (segment (start 77.1 46.55) (end 77.1 45.65) (width 0.25) (layer F.Cu) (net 6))
 (segment (start 79.3 44.7) (end 77.1 44.7) (width 0.25) (layer F.Cu) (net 5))
 (segment (start 74.075009 43.850009) (end 73.8 43.575) (width 0.2) (layer F.Cu) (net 8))
 (segment (start 72.907091 56.05002) (end 74.075009 54.882102) (width 0.2) (layer F.Cu) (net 8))
 (segment (start 70.56502 56.05002) (end 72.907091 56.05002) (width 0.2) (layer F.Cu) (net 8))
 (segment (start 74.075009 54.882102) (end 74.075009 43.850009) (width 0.2) (layer F.Cu) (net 8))
 (segment (start 69.865 55.35) (end 70.56502 56.05002) (width 0.2) (layer F.Cu) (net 8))
 (segment (start 73.8 43.575) (end 73.175 43.575) (width 0.2) (layer F.Cu) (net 8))
 (segment (start 69.865 54.55) (end 69.865 55.35) (width 0.2) (layer F.Cu) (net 8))
 (segment (start 71.425 43.575) (end 70.875 43.575) (width 0.25) (layer F.Cu) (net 10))
 (segment (start 70.6 43.3) (end 70.0875 43.3) (width 0.25) (layer F.Cu) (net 10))
 (segment (start 70.875 43.575) (end 70.6 43.3) (width 0.25) (layer F.Cu) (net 10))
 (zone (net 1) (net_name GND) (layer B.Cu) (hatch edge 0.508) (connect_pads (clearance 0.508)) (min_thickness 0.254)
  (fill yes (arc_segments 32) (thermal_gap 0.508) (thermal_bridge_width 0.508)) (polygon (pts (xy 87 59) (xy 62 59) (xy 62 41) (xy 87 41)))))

